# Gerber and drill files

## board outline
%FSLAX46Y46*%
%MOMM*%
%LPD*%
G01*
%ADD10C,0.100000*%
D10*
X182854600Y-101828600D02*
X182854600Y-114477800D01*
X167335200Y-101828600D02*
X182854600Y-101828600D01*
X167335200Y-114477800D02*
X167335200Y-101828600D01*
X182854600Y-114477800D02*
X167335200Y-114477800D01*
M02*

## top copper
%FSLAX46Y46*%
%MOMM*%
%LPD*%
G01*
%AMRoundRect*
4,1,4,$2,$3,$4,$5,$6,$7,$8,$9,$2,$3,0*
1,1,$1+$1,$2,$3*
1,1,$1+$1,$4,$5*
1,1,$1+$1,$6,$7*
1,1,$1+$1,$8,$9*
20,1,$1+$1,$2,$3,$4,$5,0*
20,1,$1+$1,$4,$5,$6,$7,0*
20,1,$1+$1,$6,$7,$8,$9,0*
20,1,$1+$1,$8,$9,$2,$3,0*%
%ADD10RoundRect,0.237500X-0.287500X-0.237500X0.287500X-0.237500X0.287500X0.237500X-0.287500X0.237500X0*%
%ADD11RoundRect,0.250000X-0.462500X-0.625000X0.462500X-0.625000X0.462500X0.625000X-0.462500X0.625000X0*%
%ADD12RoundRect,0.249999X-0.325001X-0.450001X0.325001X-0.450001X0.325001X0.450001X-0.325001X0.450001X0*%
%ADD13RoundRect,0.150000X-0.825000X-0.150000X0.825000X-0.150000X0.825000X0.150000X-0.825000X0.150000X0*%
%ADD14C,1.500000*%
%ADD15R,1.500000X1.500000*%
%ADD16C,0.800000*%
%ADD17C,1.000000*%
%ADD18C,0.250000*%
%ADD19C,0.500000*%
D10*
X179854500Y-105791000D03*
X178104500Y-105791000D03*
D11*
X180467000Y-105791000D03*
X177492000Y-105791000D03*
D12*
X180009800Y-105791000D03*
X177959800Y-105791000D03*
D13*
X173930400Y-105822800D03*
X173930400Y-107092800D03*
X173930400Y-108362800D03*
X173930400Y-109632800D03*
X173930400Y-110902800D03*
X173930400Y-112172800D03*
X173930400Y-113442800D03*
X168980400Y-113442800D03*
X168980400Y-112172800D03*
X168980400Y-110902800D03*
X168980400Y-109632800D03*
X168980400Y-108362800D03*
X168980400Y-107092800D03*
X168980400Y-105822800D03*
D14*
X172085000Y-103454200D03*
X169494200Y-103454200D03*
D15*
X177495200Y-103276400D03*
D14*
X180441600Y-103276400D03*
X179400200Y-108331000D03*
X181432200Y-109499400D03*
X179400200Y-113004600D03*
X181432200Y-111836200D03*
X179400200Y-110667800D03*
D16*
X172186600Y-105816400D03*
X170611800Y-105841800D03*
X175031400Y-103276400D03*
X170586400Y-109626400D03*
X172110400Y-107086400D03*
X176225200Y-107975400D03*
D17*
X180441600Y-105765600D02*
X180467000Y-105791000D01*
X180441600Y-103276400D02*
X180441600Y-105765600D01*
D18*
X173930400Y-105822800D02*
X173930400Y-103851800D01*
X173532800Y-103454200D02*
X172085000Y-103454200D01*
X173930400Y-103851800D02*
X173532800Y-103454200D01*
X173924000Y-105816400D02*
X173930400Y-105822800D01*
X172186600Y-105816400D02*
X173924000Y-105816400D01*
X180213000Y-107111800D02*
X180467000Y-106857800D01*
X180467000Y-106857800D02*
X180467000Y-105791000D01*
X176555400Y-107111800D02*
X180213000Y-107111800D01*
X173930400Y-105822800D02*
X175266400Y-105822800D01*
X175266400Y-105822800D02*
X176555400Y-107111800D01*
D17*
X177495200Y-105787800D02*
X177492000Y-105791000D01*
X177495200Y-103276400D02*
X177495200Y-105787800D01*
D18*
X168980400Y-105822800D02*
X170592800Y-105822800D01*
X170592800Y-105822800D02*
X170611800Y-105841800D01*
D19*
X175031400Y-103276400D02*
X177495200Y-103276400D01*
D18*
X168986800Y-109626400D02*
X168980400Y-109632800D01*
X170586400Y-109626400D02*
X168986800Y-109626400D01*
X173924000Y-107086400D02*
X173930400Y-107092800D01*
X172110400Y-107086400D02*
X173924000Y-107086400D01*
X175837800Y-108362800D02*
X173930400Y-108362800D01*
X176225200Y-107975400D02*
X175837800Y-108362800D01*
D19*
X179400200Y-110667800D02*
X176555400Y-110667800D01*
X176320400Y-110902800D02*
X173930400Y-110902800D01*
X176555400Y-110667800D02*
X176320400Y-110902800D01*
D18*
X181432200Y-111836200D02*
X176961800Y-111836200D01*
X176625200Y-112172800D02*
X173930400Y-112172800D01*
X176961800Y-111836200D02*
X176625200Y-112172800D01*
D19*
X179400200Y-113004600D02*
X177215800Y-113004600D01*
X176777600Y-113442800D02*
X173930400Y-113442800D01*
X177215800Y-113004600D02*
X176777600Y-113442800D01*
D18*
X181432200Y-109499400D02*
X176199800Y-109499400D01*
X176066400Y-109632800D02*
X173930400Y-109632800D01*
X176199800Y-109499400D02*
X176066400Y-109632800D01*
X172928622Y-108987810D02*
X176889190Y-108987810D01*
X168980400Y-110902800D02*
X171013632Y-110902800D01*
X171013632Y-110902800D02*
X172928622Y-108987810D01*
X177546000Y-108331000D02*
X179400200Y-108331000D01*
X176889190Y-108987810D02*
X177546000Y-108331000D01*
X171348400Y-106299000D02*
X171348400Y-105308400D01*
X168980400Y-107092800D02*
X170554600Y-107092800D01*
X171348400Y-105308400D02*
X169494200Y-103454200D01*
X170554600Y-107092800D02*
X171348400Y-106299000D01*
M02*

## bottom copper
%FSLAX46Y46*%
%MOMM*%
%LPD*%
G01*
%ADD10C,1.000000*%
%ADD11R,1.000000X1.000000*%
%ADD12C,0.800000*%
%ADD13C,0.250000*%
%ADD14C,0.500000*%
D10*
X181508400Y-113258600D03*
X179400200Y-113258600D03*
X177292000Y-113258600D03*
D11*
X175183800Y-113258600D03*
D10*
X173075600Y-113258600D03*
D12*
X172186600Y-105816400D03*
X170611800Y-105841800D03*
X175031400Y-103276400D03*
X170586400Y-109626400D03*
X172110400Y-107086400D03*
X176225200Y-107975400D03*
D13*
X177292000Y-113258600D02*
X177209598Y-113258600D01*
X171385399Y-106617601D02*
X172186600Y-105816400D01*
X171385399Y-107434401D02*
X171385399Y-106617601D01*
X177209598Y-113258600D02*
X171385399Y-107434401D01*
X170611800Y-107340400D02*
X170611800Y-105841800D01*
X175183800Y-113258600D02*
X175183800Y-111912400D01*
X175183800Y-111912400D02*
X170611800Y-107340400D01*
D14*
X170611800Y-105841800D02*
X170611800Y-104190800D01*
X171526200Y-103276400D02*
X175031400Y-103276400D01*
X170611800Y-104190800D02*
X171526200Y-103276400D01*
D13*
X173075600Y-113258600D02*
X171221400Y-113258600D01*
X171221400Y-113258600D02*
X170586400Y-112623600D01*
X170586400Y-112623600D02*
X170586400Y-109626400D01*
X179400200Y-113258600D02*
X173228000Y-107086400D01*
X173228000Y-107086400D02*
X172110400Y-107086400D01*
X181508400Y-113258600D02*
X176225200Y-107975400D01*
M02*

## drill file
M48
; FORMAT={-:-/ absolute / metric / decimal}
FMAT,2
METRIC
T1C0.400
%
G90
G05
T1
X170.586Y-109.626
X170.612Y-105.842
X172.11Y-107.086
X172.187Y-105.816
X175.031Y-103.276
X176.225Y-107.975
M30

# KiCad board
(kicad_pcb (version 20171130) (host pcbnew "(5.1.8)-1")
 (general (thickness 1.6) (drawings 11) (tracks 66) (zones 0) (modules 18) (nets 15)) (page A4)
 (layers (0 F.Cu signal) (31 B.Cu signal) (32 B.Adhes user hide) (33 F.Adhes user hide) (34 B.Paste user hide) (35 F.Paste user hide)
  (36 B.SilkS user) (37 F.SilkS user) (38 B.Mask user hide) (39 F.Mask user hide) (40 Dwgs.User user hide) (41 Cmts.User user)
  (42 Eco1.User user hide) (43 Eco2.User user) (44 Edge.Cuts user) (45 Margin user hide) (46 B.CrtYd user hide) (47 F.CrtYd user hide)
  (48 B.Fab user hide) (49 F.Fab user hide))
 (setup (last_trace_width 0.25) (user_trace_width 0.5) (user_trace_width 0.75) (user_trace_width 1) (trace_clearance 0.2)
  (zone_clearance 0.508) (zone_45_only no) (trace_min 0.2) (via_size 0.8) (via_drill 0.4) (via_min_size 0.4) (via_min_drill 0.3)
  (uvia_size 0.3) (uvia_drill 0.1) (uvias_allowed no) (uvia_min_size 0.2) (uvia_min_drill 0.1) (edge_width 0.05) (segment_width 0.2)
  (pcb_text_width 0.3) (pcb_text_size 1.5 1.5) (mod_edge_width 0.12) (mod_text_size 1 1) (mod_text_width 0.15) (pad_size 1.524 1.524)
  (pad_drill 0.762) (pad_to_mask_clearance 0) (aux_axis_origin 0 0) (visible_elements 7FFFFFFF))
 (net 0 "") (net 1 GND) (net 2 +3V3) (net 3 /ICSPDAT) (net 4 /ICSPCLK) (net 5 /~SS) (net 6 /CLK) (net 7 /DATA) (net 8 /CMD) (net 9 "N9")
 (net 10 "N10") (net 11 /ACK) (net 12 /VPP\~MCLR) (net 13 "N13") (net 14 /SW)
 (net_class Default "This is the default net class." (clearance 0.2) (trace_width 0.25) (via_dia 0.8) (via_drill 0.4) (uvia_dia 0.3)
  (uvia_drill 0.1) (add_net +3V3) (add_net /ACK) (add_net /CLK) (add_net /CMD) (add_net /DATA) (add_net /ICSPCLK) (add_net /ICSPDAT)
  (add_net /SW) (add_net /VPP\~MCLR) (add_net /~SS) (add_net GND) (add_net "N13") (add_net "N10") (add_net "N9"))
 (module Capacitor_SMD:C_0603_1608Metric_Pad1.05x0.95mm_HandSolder (layer F.Cu) (at 178.9795 105.791)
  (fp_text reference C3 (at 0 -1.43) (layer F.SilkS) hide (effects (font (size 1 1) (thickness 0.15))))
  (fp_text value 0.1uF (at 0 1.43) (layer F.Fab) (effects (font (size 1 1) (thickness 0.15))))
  (pad 2 smd roundrect (at 0.875 0) (size 1.05 0.95) (layers F.Cu F.Paste F.Mask) (roundrect_rratio 0.25) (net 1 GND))
  (pad 1 smd roundrect (at -0.875 0) (size 1.05 0.95) (layers F.Cu F.Paste F.Mask) (roundrect_rratio 0.25) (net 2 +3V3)))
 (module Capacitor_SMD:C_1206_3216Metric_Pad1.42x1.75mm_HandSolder (layer F.Cu) (at 178.9795 105.791)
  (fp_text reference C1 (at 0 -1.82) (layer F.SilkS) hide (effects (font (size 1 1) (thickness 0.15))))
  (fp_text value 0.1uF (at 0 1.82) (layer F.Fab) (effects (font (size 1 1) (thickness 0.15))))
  (pad 2 smd roundrect (at 1.4875 0) (size 1.425 1.75) (layers F.Cu F.Paste F.Mask) (roundrect_rratio 0.1754385964912281) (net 1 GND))
  (pad 1 smd roundrect (at -1.4875 0) (size 1.425 1.75) (layers F.Cu F.Paste F.Mask) (roundrect_rratio 0.1754385964912281) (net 2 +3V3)))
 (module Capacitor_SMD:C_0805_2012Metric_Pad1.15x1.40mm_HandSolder (layer F.Cu) (at 178.9848 105.791)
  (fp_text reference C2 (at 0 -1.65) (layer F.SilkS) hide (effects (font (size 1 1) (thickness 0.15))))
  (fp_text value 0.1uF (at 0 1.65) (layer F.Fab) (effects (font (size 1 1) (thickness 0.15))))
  (pad 2 smd roundrect (at 1.025 0) (size 1.15 1.4) (layers F.Cu F.Paste F.Mask) (roundrect_rratio 0.2173904347826087) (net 1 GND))
  (pad 1 smd roundrect (at -1.025 0) (size 1.15 1.4) (layers F.Cu F.Paste F.Mask) (roundrect_rratio 0.2173904347826087) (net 2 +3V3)))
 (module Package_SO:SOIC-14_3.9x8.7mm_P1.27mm (layer F.Cu) (at 171.4554 109.6328)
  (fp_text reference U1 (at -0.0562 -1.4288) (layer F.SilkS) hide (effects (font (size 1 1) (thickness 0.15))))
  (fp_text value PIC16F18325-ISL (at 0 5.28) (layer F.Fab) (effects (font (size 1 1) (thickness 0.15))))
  (pad 14 smd roundrect (at 2.475 -3.81) (size 1.95 0.6) (layers F.Cu F.Paste F.Mask) (roundrect_rratio 0.25) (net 1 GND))
  (pad 13 smd roundrect (at 2.475 -2.54) (size 1.95 0.6) (layers F.Cu F.Paste F.Mask) (roundrect_rratio 0.25) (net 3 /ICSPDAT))
  (pad 12 smd roundrect (at 2.475 -1.27) (size 1.95 0.6) (layers F.Cu F.Paste F.Mask) (roundrect_rratio 0.25) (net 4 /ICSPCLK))
  (pad 11 smd roundrect (at 2.475 0) (size 1.95 0.6) (layers F.Cu F.Paste F.Mask) (roundrect_rratio 0.25) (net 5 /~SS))
  (pad 10 smd roundrect (at 2.475 1.27) (size 1.95 0.6) (layers F.Cu F.Paste F.Mask) (roundrect_rratio 0.25) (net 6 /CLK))
  (pad 9 smd roundrect (at 2.475 2.54) (size 1.95 0.6) (layers F.Cu F.Paste F.Mask) (roundrect_rratio 0.25) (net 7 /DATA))
  (pad 8 smd roundrect (at 2.475 3.81) (size 1.95 0.6) (layers F.Cu F.Paste F.Mask) (roundrect_rratio 0.25) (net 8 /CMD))
  (pad 7 smd roundrect (at -2.475 3.81) (size 1.95 0.6) (layers F.Cu F.Paste F.Mask) (roundrect_rratio 0.25) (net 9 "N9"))
  (pad 6 smd roundrect (at -2.475 2.54) (size 1.95 0.6) (layers F.Cu F.Paste F.Mask) (roundrect_rratio 0.25) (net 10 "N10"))
  (pad 5 smd roundrect (at -2.475 1.27) (size 1.95 0.6) (layers F.Cu F.Paste F.Mask) (roundrect_rratio 0.25) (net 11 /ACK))
  (pad 4 smd roundrect (at -2.475 0) (size 1.95 0.6) (layers F.Cu F.Paste F.Mask) (roundrect_rratio 0.25) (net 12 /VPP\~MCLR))
  (pad 3 smd roundrect (at -2.475 -1.27) (size 1.95 0.6) (layers F.Cu F.Paste F.Mask) (roundrect_rratio 0.25) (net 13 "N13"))
  (pad 2 smd roundrect (at -2.475 -2.54) (size 1.95 0.6) (layers F.Cu F.Paste F.Mask) (roundrect_rratio 0.25) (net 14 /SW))
  (pad 1 smd roundrect (at -2.475 -3.81) (size 1.95 0.6) (layers F.Cu F.Paste F.Mask) (roundrect_rratio 0.25) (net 2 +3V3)))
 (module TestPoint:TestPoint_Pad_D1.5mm (layer F.Cu) (at 172.085 103.4542 90)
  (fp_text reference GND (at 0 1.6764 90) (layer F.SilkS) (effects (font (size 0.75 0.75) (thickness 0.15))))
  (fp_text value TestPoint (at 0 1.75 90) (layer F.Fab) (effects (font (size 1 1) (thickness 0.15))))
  (pad 1 smd circle (at 0 0 90) (size 1.5 1.5) (layers F.Cu F.Mask) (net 1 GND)))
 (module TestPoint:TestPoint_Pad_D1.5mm (layer F.Cu) (at 169.4942 103.4542 90)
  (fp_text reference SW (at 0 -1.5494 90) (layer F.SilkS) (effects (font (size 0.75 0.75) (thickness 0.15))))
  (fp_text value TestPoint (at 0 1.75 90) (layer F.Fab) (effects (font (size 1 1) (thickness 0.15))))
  (pad 1 smd circle (at 0 0 90) (size 1.5 1.5) (layers F.Cu F.Mask) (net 14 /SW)))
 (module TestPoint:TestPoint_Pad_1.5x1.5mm (layer F.Cu) (at 177.4952 103.2764 180)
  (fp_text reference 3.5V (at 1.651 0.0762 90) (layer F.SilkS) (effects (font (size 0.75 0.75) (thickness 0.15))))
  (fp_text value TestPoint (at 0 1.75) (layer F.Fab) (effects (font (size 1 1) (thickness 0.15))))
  (pad 1 smd rect (at 0 0 180) (size 1.5 1.5) (layers F.Cu F.Mask) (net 2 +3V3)))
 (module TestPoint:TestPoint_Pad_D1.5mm (layer F.Cu) (at 180.4416 103.2764)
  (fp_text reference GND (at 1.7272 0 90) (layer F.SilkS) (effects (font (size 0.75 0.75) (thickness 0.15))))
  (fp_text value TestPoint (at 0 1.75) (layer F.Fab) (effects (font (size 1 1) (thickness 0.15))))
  (pad 1 smd circle (at 0 0) (size 1.5 1.5) (layers F.Cu F.Mask) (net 1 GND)))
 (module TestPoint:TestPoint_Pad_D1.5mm (layer F.Cu) (at 179.4002 108.331)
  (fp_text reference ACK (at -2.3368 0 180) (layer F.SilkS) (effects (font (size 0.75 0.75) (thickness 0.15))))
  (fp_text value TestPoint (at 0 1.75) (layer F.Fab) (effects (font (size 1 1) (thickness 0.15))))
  (pad 1 smd circle (at 0 0) (size 1.5 1.5) (layers F.Cu F.Mask) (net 11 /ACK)))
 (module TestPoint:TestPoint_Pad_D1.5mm (layer F.Cu) (at 181.4322 109.4994)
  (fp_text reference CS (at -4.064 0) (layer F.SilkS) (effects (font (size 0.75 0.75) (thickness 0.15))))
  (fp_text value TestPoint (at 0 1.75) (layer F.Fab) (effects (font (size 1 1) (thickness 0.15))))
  (pad 1 smd circle (at 0 0) (size 1.5 1.5) (layers F.Cu F.Mask) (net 5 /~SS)))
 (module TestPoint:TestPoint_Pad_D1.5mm (layer F.Cu) (at 179.4002 113.0046)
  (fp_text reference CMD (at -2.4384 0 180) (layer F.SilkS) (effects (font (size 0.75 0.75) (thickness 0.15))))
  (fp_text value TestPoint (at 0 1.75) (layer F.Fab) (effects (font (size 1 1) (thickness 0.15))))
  (pad 1 smd circle (at 0 0) (size 1.5 1.5) (layers F.Cu F.Mask) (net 8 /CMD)))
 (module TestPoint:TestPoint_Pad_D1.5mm (layer F.Cu) (at 181.4322 111.8362)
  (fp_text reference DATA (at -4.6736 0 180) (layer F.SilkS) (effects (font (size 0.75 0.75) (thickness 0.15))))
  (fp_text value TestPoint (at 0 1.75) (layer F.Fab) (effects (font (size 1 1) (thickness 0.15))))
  (pad 1 smd circle (at 0 0) (size 1.5 1.5) (layers F.Cu F.Mask) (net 7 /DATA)))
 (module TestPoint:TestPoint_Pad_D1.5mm (layer F.Cu) (at 179.4002 110.6678)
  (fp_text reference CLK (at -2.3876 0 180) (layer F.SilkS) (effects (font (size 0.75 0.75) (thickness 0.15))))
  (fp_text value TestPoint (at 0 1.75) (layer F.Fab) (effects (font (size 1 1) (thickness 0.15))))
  (pad 1 smd circle (at 0 0) (size 1.5 1.5) (layers F.Cu F.Mask) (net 6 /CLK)))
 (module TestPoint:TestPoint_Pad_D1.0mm (layer B.Cu) (at 181.5084 113.2586 180)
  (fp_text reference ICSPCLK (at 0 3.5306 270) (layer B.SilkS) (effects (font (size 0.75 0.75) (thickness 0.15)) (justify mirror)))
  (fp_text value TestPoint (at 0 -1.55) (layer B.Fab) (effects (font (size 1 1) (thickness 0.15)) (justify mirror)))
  (pad 1 smd circle (at 0 0 180) (size 1 1) (layers B.Cu B.Mask) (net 4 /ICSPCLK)))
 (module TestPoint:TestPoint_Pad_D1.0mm (layer B.Cu) (at 179.4002 113.2586 180)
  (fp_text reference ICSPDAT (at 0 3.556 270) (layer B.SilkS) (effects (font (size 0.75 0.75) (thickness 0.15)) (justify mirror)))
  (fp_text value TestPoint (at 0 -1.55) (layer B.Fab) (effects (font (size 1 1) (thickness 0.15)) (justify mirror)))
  (pad 1 smd circle (at 0 0 180) (size 1 1) (layers B.Cu B.Mask) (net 3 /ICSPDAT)))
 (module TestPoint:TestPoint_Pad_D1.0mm (layer B.Cu) (at 177.292 113.2586 180)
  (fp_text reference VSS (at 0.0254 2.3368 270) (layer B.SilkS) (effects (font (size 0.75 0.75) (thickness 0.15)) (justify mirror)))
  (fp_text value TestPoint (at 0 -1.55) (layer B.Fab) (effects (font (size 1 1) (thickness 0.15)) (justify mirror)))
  (pad 1 smd circle (at 0 0 180) (size 1 1) (layers B.Cu B.Mask) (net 1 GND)))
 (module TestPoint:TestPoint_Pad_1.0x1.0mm (layer B.Cu) (at 175.1838 113.2586 180)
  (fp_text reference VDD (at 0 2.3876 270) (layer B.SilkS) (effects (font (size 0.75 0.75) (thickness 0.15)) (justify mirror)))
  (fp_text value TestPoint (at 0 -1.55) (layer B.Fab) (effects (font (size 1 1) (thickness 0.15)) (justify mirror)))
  (pad 1 smd rect (at 0 0 180) (size 1 1) (layers B.Cu B.Mask) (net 2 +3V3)))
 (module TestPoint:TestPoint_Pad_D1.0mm (layer B.Cu) (at 173.0756 113.2586 180)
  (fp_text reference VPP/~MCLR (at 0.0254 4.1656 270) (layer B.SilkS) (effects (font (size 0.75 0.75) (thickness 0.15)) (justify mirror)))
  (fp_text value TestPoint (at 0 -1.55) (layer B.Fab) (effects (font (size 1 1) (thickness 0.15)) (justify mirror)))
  (pad 1 smd circle (at 0 0 180) (size 1 1) (layers B.Cu B.Mask) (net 12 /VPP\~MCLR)))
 (gr_line (start 182.8546 101.8286) (end 182.8546 114.4778) (layer Edge.Cuts) (width 0.1))
 (gr_line (start 167.3352 101.8286) (end 182.8546 101.8286) (layer Edge.Cuts) (width 0.1))
 (gr_line (start 167.3352 114.4778) (end 167.3352 101.8286) (layer Edge.Cuts) (width 0.1))
 (gr_line (start 182.8546 114.4778) (end 167.3352 114.4778) (layer Edge.Cuts) (width 0.1))
 (segment (start 180.4416 105.7656) (end 180.467 105.791) (width 1) (layer F.Cu) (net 1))
 (segment (start 180.4416 103.2764) (end 180.4416 105.7656) (width 1) (layer F.Cu) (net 1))
 (segment (start 173.9304 105.8228) (end 173.9304 103.8518) (width 0.25) (layer F.Cu) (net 1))
 (segment (start 173.5328 103.4542) (end 172.085 103.4542) (width 0.25) (layer F.Cu) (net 1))
 (segment (start 173.9304 103.8518) (end 173.5328 103.4542) (width 0.25) (layer F.Cu) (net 1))
 (via (at 172.1866 105.8164) (size 0.8) (drill 0.4) (layers F.Cu B.Cu) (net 1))
 (segment (start 177.292 113.2586) (end 177.209598 113.2586) (width 0.25) (layer B.Cu) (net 1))
 (segment (start 171.385399 106.617601) (end 172.1866 105.8164) (width 0.25) (layer B.Cu) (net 1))
 (segment (start 171.385399 107.434401) (end 171.385399 106.617601) (width 0.25) (layer B.Cu) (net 1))
 (segment (start 177.209598 113.2586) (end 171.385399 107.434401) (width 0.25) (layer B.Cu) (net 1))
 (segment (start 173.924 105.8164) (end 173.9304 105.8228) (width 0.25) (layer F.Cu) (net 1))
 (segment (start 172.1866 105.8164) (end 173.924 105.8164) (width 0.25) (layer F.Cu) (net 1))
 (segment (start 180.213 107.1118) (end 180.467 106.8578) (width 0.25) (layer F.Cu) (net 1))
 (segment (start 180.467 106.8578) (end 180.467 105.791) (width 0.25) (layer F.Cu) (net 1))
 (segment (start 176.5554 107.1118) (end 180.213 107.1118) (width 0.25) (layer F.Cu) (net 1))
 (segment (start 173.9304 105.8228) (end 175.2664 105.8228) (width 0.25) (layer F.Cu) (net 1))
 (segment (start 175.2664 105.8228) (end 176.5554 107.1118) (width 0.25) (layer F.Cu) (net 1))
 (segment (start 177.4952 105.7878) (end 177.492 105.791) (width 1) (layer F.Cu) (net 2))
 (segment (start 177.4952 103.2764) (end 177.4952 105.7878) (width 1) (layer F.Cu) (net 2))
 (via (at 170.6118 105.8418) (size 0.8) (drill 0.4) (layers F.Cu B.Cu) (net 2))
 (segment (start 168.9804 105.8228) (end 170.5928 105.8228) (width 0.25) (layer F.Cu) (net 2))
 (segment (start 170.5928 105.8228) (end 170.6118 105.8418) (width 0.25) (layer F.Cu) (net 2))
 (via (at 175.0314 103.2764) (size 0.8) (drill 0.4) (layers F.Cu B.Cu) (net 2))
 (segment (start 175.0314 103.2764) (end 177.4952 103.2764) (width 0.5) (layer F.Cu) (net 2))
 (segment (start 170.6118 107.3404) (end 170.6118 105.8418) (width 0.25) (layer B.Cu) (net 2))
 (segment (start 175.1838 113.2586) (end 175.1838 111.9124) (width 0.25) (layer B.Cu) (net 2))
 (segment (start 175.1838 111.9124) (end 170.6118 107.3404) (width 0.25) (layer B.Cu) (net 2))
 (segment (start 170.6118 105.8418) (end 170.6118 104.1908) (width 0.5) (layer B.Cu) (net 2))
 (segment (start 171.5262 103.2764) (end 175.0314 103.2764) (width 0.5) (layer B.Cu) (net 2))
 (segment (start 170.6118 104.1908) (end 171.5262 103.2764) (width 0.5) (layer B.Cu) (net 2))
 (segment (start 173.0756 113.2586) (end 171.2214 113.2586) (width 0.25) (layer B.Cu) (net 12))
 (via (at 170.5864 109.6264) (size 0.8) (drill 0.4) (layers F.Cu B.Cu) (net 12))
 (segment (start 171.2214 113.2586) (end 170.5864 112.6236) (width 0.25) (layer B.Cu) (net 12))
 (segment (start 170.5864 112.6236) (end 170.5864 109.6264) (width 0.25) (layer B.Cu) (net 12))
 (segment (start 168.9868 109.6264) (end 168.9804 109.6328) (width 0.25) (layer F.Cu) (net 12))
 (segment (start 170.5864 109.6264) (end 168.9868 109.6264) (width 0.25) (layer F.Cu) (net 12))
 (via (at 172.1104 107.0864) (size 0.8) (drill 0.4) (layers F.Cu B.Cu) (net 3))
 (segment (start 179.4002 113.2586) (end 173.228 107.0864) (width 0.25) (layer B.Cu) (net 3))
 (segment (start 173.228 107.0864) (end 172.1104 107.0864) (width 0.25) (layer B.Cu) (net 3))
 (segment (start 173.924 107.0864) (end 173.9304 107.0928) (width 0.25) (layer F.Cu) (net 3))
 (segment (start 172.1104 107.0864) (end 173.924 107.0864) (width 0.25) (layer F.Cu) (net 3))
 (via (at 176.2252 107.9754) (size 0.8) (drill 0.4) (layers F.Cu B.Cu) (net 4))
 (segment (start 181.5084 113.2586) (end 176.2252 107.9754) (width 0.25) (layer B.Cu) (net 4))
 (segment (start 175.8378 108.3628) (end 173.9304 108.3628) (width 0.25) (layer F.Cu) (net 4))
 (segment (start 176.2252 107.9754) (end 175.8378 108.3628) (width 0.25) (layer F.Cu) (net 4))
 (segment (start 179.4002 110.6678) (end 176.5554 110.6678) (width 0.5) (layer F.Cu) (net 6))
 (segment (start 176.3204 110.9028) (end 173.9304 110.9028) (width 0.5) (layer F.Cu) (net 6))
 (segment (start 176.5554 110.6678) (end 176.3204 110.9028) (width 0.5) (layer F.Cu) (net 6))
 (segment (start 181.4322 111.8362) (end 176.9618 111.8362) (width 0.25) (layer F.Cu) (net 7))
 (segment (start 176.6252 112.1728) (end 173.9304 112.1728) (width 0.25) (layer F.Cu) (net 7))
 (segment (start 176.9618 111.8362) (end 176.6252 112.1728) (width 0.25) (layer F.Cu) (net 7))
 (segment (start 179.4002 113.0046) (end 177.2158 113.0046) (width 0.5) (layer F.Cu) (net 8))
 (segment (start 176.7776 113.4428) (end 173.9304 113.4428) (width 0.5) (layer F.Cu) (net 8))
 (segment (start 177.2158 113.0046) (end 176.7776 113.4428) (width 0.5) (layer F.Cu) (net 8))
 (segment (start 181.4322 109.4994) (end 176.1998 109.4994) (width 0.25) (layer F.Cu) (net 5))
 (segment (start 176.0664 109.6328) (end 173.9304 109.6328) (width 0.25) (layer F.Cu) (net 5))
 (segment (start 176.1998 109.4994) (end 176.0664 109.6328) (width 0.25) (layer F.Cu) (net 5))
 (segment (start 172.928622 108.98781) (end 176.88919 108.98781) (width 0.25) (layer F.Cu) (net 11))
 (segment (start 168.9804 110.9028) (end 171.013632 110.9028) (width 0.25) (layer F.Cu) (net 11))
 (segment (start 171.013632 110.9028) (end 172.928622 108.98781) (width 0.25) (layer F.Cu) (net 11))
 (segment (start 177.546 108.331) (end 179.4002 108.331) (width 0.25) (layer F.Cu) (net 11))
 (segment (start 176.88919 108.98781) (end 177.546 108.331) (width 0.25) (layer F.Cu) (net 11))
 (segment (start 171.3484 106.299) (end 171.3484 105.3084) (width 0.25) (layer F.Cu) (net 14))
 (segment (start 168.9804 107.0928) (end 170.5546 107.0928) (width 0.25) (layer F.Cu) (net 14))
 (segment (start 171.3484 105.3084) (end 169.4942 103.4542) (width 0.25) (layer F.Cu) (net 14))
 (segment (start 170.5546 107.0928) (end 171.3484 106.299) (width 0.25) (layer F.Cu) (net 14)))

